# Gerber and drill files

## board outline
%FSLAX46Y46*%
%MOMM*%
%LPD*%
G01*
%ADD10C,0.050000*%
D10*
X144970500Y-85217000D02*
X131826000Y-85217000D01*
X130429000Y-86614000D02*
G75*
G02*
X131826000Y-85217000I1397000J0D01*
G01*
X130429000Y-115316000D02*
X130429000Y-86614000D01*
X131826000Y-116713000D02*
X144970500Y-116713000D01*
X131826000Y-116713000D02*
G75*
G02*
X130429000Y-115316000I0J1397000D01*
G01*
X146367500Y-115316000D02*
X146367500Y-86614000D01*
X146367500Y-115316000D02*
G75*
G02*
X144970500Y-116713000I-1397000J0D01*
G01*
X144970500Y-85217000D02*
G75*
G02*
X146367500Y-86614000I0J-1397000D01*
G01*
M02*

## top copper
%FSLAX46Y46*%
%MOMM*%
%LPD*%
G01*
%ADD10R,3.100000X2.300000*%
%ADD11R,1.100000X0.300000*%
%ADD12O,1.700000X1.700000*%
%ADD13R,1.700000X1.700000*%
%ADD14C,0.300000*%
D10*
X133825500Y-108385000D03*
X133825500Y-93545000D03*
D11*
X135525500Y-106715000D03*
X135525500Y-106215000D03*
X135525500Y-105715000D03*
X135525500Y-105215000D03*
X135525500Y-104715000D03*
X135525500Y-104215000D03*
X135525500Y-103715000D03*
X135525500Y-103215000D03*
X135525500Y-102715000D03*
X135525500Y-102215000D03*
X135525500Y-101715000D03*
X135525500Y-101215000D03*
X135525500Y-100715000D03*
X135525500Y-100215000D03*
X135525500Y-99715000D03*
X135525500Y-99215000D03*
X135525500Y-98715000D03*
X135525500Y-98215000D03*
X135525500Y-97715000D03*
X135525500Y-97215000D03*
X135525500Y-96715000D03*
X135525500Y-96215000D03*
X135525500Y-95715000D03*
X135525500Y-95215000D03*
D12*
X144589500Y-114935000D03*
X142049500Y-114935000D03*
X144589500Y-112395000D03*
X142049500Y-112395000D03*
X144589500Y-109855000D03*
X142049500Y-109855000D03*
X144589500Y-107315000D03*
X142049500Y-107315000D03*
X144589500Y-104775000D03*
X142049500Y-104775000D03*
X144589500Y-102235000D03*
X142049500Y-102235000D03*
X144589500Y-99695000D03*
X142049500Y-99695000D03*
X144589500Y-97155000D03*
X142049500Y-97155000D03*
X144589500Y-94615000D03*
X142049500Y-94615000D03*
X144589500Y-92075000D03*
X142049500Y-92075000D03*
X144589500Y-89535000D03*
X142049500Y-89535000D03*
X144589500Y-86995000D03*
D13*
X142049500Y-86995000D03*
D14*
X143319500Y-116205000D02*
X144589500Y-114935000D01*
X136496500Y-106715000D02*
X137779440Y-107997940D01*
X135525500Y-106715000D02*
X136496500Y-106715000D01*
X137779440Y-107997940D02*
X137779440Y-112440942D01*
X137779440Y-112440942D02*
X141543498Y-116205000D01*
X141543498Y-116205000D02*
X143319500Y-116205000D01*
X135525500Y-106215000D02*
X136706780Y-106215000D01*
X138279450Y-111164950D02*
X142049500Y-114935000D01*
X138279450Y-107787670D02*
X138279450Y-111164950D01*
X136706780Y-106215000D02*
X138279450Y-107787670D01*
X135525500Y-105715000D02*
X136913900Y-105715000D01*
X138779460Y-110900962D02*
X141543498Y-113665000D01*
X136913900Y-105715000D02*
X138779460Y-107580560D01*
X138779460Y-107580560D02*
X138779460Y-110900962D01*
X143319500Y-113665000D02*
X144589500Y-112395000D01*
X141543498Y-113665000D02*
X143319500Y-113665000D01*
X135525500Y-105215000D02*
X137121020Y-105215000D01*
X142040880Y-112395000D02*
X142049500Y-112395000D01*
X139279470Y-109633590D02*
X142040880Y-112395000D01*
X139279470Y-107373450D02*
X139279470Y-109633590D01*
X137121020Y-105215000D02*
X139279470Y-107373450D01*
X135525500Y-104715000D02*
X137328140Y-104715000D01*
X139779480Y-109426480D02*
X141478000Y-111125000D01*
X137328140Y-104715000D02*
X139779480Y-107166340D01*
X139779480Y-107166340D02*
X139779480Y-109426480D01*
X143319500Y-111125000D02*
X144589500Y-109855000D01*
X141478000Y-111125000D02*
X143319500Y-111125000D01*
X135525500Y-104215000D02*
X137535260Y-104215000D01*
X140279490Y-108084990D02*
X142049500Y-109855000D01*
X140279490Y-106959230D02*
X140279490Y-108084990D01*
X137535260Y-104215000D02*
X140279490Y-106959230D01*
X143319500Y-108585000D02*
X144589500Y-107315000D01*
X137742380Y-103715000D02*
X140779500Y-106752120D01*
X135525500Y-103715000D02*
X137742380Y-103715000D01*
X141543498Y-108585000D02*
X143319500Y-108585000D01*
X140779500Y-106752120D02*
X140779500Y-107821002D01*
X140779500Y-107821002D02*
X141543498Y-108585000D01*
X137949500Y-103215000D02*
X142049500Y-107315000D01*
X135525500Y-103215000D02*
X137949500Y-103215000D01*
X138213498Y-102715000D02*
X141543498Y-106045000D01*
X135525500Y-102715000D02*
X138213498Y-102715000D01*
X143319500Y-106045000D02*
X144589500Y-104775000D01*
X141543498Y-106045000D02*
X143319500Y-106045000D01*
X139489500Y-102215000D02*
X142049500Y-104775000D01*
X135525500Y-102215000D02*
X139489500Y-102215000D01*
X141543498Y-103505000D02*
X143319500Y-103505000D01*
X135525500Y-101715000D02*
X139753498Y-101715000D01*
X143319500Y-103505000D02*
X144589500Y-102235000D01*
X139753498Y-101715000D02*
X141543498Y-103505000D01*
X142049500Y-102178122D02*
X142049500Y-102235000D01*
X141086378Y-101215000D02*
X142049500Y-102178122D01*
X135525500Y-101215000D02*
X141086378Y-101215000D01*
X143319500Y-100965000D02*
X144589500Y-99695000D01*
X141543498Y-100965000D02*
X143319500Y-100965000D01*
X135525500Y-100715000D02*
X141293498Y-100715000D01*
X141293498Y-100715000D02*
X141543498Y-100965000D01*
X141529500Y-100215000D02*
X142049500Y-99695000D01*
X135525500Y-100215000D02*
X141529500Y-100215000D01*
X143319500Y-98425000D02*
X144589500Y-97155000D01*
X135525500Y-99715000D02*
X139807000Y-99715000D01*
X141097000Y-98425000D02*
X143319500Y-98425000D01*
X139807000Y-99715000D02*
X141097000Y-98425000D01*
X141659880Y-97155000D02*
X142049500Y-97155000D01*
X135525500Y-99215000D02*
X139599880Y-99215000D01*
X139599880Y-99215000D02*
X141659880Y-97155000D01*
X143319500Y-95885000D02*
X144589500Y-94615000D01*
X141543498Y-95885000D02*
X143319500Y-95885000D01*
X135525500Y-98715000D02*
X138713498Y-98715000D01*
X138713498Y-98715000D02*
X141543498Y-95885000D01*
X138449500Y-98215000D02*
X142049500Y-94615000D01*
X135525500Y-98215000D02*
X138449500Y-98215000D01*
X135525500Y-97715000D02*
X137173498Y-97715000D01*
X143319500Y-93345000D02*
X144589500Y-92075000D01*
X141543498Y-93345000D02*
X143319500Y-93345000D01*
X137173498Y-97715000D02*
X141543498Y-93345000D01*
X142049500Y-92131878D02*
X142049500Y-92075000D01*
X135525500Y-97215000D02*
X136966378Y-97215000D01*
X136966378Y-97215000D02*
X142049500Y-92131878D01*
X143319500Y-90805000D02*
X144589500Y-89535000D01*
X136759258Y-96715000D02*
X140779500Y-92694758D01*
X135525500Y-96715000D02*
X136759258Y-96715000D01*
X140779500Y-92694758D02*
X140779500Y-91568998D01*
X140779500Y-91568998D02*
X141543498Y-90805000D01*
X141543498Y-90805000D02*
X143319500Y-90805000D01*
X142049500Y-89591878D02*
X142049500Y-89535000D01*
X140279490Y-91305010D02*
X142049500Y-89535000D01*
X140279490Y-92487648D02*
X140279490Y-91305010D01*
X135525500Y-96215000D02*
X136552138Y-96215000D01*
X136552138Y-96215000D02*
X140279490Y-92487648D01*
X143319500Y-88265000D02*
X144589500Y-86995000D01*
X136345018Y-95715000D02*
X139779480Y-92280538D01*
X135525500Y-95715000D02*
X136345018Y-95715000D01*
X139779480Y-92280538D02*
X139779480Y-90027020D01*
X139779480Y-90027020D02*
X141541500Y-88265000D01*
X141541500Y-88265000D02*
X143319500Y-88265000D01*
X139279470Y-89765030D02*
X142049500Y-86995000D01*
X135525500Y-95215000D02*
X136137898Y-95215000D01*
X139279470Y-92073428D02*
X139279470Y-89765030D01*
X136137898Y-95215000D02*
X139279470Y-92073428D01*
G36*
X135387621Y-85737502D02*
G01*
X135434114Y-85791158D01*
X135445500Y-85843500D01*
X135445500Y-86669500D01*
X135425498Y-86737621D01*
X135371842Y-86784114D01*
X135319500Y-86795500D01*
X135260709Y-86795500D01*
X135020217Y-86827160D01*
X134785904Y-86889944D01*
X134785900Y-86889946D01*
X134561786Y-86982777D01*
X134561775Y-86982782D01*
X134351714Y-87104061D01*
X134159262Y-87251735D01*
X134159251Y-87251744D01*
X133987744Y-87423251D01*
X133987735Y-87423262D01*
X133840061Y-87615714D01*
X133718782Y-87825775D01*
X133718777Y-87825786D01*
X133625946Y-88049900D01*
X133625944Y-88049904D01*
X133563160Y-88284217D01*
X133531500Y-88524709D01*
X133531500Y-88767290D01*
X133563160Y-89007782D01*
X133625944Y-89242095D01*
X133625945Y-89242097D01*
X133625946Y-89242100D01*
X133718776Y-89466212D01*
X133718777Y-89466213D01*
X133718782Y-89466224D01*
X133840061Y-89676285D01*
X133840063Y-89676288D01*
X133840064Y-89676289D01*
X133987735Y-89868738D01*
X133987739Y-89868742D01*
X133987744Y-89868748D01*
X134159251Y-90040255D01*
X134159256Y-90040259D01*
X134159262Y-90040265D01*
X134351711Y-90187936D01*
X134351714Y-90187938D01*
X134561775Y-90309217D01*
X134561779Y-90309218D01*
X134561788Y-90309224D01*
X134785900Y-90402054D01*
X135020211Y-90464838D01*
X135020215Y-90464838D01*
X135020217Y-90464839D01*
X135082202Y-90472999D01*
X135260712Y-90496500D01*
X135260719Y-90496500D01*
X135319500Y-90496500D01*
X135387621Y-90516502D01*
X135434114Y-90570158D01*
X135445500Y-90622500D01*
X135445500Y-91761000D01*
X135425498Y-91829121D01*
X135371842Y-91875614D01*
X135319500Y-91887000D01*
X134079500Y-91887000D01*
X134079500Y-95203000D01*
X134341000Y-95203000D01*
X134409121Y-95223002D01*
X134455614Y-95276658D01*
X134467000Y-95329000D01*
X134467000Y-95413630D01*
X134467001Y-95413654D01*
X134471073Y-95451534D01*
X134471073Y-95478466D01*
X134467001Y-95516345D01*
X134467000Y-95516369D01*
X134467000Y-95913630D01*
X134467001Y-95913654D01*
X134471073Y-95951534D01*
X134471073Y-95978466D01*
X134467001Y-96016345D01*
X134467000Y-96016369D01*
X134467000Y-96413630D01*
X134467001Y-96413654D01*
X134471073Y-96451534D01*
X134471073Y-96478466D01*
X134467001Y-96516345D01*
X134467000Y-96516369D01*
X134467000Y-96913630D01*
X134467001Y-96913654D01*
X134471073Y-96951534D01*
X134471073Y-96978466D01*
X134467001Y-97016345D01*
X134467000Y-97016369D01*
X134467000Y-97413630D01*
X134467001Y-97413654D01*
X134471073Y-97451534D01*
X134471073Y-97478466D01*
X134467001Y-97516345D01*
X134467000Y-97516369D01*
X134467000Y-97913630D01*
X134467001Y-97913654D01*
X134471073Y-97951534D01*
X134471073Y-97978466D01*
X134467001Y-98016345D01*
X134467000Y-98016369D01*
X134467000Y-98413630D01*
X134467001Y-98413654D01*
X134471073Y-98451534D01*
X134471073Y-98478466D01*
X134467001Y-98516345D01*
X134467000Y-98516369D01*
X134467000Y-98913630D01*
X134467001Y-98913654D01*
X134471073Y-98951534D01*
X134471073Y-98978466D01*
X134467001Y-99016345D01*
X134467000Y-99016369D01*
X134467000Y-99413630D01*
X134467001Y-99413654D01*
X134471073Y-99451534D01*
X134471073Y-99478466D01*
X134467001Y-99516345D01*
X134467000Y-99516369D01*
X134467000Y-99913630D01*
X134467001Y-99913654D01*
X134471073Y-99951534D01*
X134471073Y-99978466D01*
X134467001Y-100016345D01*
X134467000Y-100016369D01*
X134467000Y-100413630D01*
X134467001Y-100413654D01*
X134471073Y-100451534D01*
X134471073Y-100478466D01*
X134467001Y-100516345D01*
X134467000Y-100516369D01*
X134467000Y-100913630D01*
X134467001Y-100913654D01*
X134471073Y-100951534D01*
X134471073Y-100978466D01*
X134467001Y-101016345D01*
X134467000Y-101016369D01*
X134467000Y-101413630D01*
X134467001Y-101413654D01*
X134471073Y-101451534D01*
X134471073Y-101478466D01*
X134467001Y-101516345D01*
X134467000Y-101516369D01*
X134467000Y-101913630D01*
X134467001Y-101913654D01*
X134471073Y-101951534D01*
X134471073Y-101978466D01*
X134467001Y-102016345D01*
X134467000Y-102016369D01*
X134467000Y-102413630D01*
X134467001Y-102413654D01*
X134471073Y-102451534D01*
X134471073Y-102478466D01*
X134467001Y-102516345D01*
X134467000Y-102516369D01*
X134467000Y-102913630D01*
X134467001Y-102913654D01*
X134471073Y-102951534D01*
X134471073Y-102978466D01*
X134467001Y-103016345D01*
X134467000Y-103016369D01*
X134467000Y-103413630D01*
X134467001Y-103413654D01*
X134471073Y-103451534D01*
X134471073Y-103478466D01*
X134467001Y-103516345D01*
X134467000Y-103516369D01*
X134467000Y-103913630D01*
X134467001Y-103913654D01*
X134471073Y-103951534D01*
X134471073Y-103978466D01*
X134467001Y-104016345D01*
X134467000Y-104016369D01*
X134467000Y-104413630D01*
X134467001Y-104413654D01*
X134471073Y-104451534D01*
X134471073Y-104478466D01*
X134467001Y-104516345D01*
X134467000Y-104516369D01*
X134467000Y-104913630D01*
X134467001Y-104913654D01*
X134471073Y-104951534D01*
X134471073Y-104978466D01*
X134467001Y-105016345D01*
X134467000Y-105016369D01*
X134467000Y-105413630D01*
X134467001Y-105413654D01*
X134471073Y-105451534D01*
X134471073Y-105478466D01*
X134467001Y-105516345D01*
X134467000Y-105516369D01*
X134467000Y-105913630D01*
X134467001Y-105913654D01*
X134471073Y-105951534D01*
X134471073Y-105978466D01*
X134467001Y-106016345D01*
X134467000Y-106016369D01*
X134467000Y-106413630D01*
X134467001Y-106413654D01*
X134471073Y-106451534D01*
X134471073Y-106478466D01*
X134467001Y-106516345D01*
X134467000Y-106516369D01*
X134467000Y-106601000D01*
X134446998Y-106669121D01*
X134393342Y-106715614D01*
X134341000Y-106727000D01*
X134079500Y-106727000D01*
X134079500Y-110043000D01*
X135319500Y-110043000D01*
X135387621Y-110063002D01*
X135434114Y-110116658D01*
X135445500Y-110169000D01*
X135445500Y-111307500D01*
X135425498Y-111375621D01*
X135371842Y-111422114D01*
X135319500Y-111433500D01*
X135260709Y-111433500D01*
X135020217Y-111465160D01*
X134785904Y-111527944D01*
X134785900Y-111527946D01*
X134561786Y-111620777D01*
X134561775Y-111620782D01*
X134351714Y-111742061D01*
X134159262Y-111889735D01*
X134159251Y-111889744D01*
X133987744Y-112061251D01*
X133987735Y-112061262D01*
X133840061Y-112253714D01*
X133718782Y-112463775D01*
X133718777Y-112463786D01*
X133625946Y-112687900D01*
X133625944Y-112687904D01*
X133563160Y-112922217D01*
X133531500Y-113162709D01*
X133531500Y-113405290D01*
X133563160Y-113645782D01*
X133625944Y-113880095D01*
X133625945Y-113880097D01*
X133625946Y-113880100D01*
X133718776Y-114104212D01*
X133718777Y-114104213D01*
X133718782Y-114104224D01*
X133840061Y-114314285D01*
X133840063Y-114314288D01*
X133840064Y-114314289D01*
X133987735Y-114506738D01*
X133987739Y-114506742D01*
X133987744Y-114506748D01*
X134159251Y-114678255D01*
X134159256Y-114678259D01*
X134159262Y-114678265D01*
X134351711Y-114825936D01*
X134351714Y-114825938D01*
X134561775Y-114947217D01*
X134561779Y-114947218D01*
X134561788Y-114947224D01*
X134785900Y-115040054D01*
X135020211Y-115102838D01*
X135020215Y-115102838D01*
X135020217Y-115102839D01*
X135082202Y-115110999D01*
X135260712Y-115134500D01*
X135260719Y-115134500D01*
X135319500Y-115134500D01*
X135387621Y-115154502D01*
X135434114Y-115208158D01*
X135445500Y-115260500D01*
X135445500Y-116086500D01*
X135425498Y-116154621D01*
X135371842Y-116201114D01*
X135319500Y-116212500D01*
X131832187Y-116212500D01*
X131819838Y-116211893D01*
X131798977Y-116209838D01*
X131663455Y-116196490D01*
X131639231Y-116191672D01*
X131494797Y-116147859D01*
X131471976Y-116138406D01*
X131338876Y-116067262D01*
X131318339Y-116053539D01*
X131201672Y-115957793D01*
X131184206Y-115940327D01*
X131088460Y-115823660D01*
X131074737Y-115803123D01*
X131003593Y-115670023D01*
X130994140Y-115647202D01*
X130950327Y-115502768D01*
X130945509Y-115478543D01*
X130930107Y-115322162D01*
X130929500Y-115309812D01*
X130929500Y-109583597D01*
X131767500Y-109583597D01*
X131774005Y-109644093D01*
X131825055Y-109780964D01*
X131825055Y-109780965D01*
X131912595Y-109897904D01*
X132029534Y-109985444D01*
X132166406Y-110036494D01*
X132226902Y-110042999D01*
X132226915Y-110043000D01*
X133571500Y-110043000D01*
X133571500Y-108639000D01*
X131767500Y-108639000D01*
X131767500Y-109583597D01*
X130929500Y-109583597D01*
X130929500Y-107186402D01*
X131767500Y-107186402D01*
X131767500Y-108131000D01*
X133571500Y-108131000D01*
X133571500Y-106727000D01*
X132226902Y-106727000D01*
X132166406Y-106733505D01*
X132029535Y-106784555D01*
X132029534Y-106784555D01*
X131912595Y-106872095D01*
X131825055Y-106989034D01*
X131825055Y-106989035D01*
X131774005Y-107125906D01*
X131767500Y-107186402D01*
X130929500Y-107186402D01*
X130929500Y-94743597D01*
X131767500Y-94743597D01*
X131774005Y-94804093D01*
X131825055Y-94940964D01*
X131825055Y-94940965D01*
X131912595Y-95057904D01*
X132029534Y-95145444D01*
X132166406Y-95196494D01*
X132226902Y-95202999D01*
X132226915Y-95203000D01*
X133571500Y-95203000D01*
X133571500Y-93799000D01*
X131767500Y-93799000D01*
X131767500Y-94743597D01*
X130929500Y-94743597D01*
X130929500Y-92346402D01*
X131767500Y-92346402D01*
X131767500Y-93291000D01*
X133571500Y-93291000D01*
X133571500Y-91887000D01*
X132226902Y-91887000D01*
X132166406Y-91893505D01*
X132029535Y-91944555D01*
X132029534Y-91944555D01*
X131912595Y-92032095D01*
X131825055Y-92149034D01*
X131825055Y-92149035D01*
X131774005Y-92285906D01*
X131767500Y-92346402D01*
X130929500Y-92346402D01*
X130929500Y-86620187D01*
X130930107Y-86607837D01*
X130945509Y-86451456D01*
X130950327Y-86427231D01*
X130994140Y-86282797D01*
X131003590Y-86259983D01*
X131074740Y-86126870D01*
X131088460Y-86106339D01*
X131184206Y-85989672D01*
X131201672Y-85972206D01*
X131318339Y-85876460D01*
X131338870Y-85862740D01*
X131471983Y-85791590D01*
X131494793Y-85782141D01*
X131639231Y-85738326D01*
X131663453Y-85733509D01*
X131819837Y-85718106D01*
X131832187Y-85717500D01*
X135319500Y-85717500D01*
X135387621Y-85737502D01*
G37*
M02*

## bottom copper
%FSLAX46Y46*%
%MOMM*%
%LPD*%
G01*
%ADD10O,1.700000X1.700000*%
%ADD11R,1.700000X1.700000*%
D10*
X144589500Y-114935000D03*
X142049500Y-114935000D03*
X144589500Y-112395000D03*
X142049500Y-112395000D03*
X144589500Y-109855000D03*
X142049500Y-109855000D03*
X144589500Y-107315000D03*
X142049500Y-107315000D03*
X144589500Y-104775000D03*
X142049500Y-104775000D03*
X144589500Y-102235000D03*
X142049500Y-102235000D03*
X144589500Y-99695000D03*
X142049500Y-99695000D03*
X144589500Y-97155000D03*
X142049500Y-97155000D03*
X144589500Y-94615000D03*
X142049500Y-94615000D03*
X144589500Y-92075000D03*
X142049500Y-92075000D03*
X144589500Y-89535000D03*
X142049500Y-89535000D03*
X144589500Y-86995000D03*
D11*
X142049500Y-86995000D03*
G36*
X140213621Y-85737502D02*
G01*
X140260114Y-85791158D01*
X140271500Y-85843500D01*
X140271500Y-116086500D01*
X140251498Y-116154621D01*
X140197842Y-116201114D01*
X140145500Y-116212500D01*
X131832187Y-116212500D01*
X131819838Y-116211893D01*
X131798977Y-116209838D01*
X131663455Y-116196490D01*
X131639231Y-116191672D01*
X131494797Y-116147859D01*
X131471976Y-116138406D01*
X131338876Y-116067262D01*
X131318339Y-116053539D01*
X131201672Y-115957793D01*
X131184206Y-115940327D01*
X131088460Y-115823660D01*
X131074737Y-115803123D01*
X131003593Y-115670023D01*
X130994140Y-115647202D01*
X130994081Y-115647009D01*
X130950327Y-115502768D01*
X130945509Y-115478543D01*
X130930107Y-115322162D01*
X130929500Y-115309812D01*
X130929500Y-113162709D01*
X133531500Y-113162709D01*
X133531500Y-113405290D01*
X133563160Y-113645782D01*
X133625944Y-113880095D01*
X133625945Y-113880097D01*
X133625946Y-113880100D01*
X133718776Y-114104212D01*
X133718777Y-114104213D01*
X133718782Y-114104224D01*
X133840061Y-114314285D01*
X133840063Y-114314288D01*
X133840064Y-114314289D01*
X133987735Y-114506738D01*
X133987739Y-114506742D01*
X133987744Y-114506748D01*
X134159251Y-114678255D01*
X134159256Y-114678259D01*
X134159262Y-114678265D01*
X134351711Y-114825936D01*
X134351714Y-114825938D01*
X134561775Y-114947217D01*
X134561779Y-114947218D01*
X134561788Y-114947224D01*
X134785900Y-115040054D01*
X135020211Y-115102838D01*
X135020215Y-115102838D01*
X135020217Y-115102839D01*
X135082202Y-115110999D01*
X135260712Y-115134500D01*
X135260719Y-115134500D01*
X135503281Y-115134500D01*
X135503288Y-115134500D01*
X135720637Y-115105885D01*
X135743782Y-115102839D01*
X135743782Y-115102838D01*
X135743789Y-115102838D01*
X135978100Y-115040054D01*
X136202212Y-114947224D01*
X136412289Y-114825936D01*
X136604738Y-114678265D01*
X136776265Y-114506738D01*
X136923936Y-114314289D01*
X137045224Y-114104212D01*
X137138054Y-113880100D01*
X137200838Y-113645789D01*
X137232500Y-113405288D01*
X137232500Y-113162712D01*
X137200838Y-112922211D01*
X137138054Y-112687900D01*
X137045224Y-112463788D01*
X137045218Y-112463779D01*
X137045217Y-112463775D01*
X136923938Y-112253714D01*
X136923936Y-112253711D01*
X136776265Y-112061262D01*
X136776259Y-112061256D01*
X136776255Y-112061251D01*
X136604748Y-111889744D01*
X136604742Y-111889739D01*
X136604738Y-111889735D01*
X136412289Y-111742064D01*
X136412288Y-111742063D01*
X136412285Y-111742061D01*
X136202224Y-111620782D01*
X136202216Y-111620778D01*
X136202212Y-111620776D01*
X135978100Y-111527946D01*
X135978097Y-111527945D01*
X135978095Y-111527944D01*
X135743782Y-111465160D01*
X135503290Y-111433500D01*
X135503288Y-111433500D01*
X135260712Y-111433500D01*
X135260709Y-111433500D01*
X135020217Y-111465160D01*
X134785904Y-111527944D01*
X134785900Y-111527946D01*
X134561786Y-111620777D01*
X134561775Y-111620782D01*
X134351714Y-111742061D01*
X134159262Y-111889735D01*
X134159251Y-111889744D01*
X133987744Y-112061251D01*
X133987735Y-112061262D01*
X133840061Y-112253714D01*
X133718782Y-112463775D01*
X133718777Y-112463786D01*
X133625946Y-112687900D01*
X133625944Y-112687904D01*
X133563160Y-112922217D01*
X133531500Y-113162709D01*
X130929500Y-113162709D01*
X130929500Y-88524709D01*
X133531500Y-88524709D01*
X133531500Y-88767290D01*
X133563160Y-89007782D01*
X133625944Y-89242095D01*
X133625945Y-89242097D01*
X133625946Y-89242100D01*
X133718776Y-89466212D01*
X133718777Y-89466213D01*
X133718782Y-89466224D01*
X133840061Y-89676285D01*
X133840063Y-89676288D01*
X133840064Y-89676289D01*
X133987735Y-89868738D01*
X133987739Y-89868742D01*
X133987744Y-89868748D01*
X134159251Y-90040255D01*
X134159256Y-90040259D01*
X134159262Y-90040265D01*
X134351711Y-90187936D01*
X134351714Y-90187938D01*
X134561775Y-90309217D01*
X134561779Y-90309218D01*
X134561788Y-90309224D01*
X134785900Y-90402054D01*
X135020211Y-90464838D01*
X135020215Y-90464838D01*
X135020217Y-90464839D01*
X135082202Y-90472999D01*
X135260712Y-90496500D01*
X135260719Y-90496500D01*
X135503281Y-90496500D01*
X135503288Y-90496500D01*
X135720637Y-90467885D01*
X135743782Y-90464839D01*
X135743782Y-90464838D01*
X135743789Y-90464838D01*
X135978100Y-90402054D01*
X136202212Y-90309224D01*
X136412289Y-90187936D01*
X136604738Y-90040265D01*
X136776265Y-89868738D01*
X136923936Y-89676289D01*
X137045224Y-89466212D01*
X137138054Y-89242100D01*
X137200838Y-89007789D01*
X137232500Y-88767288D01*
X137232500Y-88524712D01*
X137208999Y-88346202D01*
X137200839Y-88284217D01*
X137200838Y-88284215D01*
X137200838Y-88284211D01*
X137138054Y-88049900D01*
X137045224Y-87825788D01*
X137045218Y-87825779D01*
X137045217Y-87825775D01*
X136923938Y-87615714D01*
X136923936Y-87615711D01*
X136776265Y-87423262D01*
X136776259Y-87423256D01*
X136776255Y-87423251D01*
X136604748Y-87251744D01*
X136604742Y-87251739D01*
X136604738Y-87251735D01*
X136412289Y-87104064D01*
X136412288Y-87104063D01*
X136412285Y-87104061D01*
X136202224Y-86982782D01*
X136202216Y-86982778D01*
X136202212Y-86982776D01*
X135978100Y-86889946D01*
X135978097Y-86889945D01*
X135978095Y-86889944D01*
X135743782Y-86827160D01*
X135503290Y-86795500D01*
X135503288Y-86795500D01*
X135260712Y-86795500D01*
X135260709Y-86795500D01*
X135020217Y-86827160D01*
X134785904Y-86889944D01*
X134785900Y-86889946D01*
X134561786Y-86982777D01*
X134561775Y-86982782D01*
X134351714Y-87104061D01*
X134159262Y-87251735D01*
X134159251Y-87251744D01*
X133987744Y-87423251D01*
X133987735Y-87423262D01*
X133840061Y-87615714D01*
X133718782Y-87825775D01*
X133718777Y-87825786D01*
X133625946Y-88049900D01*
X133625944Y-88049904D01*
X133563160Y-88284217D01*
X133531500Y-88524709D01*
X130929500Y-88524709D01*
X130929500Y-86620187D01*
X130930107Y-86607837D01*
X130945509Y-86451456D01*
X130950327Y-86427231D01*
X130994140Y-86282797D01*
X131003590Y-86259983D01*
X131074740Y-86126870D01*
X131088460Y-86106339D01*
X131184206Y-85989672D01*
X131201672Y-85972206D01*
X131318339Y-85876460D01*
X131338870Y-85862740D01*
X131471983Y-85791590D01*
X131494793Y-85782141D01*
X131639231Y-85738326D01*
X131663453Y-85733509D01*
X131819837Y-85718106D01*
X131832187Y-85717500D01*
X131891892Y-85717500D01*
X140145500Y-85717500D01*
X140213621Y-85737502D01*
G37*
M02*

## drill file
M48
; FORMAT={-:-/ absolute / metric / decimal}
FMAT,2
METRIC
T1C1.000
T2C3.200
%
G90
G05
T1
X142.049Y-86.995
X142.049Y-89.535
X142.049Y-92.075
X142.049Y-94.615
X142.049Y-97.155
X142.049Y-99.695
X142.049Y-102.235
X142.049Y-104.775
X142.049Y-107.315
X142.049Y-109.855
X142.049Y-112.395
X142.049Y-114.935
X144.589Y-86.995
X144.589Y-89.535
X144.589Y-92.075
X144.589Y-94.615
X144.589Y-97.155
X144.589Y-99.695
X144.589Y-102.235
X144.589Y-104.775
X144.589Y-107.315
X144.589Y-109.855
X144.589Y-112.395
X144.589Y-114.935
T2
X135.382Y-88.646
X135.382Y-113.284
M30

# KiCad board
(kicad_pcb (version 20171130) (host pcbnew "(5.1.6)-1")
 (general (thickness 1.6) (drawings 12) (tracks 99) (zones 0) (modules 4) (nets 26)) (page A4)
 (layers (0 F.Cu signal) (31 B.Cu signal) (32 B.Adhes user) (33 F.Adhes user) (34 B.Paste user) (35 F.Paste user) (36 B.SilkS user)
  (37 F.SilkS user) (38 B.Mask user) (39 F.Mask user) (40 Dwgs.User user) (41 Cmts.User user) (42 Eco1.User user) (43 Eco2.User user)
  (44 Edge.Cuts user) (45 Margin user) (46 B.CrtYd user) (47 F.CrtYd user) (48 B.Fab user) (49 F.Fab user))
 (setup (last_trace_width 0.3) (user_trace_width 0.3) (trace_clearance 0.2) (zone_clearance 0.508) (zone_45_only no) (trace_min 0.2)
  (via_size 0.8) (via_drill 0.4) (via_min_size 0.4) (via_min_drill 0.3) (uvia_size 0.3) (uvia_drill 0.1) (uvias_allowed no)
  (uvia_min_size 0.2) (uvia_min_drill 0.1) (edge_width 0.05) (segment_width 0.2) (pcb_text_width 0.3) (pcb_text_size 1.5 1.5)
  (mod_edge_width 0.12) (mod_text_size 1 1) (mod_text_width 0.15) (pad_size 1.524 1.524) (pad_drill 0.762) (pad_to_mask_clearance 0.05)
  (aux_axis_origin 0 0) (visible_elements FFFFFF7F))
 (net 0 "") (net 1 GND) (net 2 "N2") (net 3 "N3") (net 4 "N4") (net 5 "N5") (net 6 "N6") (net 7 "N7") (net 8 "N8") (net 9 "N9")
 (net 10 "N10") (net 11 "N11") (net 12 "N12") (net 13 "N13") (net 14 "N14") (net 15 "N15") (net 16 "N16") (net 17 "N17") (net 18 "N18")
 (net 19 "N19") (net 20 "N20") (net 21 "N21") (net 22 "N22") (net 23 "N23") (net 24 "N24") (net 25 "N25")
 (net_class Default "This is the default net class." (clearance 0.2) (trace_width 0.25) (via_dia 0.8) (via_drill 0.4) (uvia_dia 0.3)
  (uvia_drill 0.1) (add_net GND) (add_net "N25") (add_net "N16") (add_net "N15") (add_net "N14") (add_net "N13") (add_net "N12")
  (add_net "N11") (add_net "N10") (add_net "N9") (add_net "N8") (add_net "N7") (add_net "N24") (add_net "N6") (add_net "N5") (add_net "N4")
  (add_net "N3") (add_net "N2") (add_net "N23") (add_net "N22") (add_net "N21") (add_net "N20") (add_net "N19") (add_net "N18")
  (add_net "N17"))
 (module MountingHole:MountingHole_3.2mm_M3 (layer F.Cu) (at 135.382 113.284)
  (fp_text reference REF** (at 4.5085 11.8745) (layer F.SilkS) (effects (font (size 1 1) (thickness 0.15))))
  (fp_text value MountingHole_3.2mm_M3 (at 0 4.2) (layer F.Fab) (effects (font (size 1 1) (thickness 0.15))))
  (pad 1 np_thru_hole circle (at 0 0) (size 3.2 3.2) (drill 3.2) (layers *.Cu *.Mask)))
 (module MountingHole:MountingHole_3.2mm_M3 (layer F.Cu) (at 135.382 88.646)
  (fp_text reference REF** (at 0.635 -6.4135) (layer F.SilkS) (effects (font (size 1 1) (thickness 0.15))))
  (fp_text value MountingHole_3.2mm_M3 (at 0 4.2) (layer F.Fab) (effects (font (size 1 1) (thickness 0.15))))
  (pad 1 np_thru_hole circle (at 0 0) (size 3.2 3.2) (drill 3.2) (layers *.Cu *.Mask)))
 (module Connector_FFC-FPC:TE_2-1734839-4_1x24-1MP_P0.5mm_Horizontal (layer F.Cu) (at 134.1755 100.965 270)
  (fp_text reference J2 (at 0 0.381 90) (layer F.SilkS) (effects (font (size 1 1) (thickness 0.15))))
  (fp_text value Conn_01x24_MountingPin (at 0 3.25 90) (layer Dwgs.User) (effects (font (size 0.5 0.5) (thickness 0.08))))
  (pad MP smd rect (at 7.42 0.35 270) (size 2.3 3.1) (layers F.Cu F.Paste F.Mask) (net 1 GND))
  (pad MP smd rect (at -7.42 0.35 270) (size 2.3 3.1) (layers F.Cu F.Paste F.Mask) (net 1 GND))
  (pad 24 smd rect (at 5.75 -1.35 270) (size 0.3 1.1) (layers F.Cu F.Paste F.Mask) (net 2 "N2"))
  (pad 23 smd rect (at 5.25 -1.35 270) (size 0.3 1.1) (layers F.Cu F.Paste F.Mask) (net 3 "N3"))
  (pad 22 smd rect (at 4.75 -1.35 270) (size 0.3 1.1) (layers F.Cu F.Paste F.Mask) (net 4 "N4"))
  (pad 21 smd rect (at 4.25 -1.35 270) (size 0.3 1.1) (layers F.Cu F.Paste F.Mask) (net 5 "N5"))
  (pad 20 smd rect (at 3.75 -1.35 270) (size 0.3 1.1) (layers F.Cu F.Paste F.Mask) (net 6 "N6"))
  (pad 19 smd rect (at 3.25 -1.35 270) (size 0.3 1.1) (layers F.Cu F.Paste F.Mask) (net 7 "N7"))
  (pad 18 smd rect (at 2.75 -1.35 270) (size 0.3 1.1) (layers F.Cu F.Paste F.Mask) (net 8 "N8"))
  (pad 17 smd rect (at 2.25 -1.35 270) (size 0.3 1.1) (layers F.Cu F.Paste F.Mask) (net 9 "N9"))
  (pad 16 smd rect (at 1.75 -1.35 270) (size 0.3 1.1) (layers F.Cu F.Paste F.Mask) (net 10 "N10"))
  (pad 15 smd rect (at 1.25 -1.35 270) (size 0.3 1.1) (layers F.Cu F.Paste F.Mask) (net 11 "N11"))
  (pad 14 smd rect (at 0.75 -1.35 270) (size 0.3 1.1) (layers F.Cu F.Paste F.Mask) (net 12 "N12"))
  (pad 13 smd rect (at 0.25 -1.35 270) (size 0.3 1.1) (layers F.Cu F.Paste F.Mask) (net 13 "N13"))
  (pad 12 smd rect (at -0.25 -1.35 270) (size 0.3 1.1) (layers F.Cu F.Paste F.Mask) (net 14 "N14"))
  (pad 11 smd rect (at -0.75 -1.35 270) (size 0.3 1.1) (layers F.Cu F.Paste F.Mask) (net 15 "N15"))
  (pad 10 smd rect (at -1.25 -1.35 270) (size 0.3 1.1) (layers F.Cu F.Paste F.Mask) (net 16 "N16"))
  (pad 9 smd rect (at -1.75 -1.35 270) (size 0.3 1.1) (layers F.Cu F.Paste F.Mask) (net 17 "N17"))
  (pad 8 smd rect (at -2.25 -1.35 270) (size 0.3 1.1) (layers F.Cu F.Paste F.Mask) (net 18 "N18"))
  (pad 7 smd rect (at -2.75 -1.35 270) (size 0.3 1.1) (layers F.Cu F.Paste F.Mask) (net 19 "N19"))
  (pad 6 smd rect (at -3.25 -1.35 270) (size 0.3 1.1) (layers F.Cu F.Paste F.Mask) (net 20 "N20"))
  (pad 5 smd rect (at -3.75 -1.35 270) (size 0.3 1.1) (layers F.Cu F.Paste F.Mask) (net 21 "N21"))
  (pad 4 smd rect (at -4.25 -1.35 270) (size 0.3 1.1) (layers F.Cu F.Paste F.Mask) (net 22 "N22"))
  (pad 3 smd rect (at -4.75 -1.35 270) (size 0.3 1.1) (layers F.Cu F.Paste F.Mask) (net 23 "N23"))
  (pad 2 smd rect (at -5.25 -1.35 270) (size 0.3 1.1) (layers F.Cu F.Paste F.Mask) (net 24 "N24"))
  (pad 1 smd rect (at -5.75 -1.35 270) (size 0.3 1.1) (layers F.Cu F.Paste F.Mask) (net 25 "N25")))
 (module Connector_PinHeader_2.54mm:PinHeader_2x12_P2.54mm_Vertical (layer F.Cu) (at 142.0495 86.995)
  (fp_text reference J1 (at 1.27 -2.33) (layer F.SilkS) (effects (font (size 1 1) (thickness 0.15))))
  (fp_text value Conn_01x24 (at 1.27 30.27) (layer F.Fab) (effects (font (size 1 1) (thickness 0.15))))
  (pad 24 thru_hole oval (at 2.54 27.94) (size 1.7 1.7) (drill 1) (layers *.Cu *.Mask) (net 2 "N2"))
  (pad 23 thru_hole oval (at 0 27.94) (size 1.7 1.7) (drill 1) (layers *.Cu *.Mask) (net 3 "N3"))
  (pad 22 thru_hole oval (at 2.54 25.4) (size 1.7 1.7) (drill 1) (layers *.Cu *.Mask) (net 4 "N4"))
  (pad 21 thru_hole oval (at 0 25.4) (size 1.7 1.7) (drill 1) (layers *.Cu *.Mask) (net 5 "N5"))
  (pad 20 thru_hole oval (at 2.54 22.86) (size 1.7 1.7) (drill 1) (layers *.Cu *.Mask) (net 6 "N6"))
  (pad 19 thru_hole oval (at 0 22.86) (size 1.7 1.7) (drill 1) (layers *.Cu *.Mask) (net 7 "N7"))
  (pad 18 thru_hole oval (at 2.54 20.32) (size 1.7 1.7) (drill 1) (layers *.Cu *.Mask) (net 8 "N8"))
  (pad 17 thru_hole oval (at 0 20.32) (size 1.7 1.7) (drill 1) (layers *.Cu *.Mask) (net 9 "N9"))
  (pad 16 thru_hole oval (at 2.54 17.78) (size 1.7 1.7) (drill 1) (layers *.Cu *.Mask) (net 10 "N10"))
  (pad 15 thru_hole oval (at 0 17.78) (size 1.7 1.7) (drill 1) (layers *.Cu *.Mask) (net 11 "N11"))
  (pad 14 thru_hole oval (at 2.54 15.24) (size 1.7 1.7) (drill 1) (layers *.Cu *.Mask) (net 12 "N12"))
  (pad 13 thru_hole oval (at 0 15.24) (size 1.7 1.7) (drill 1) (layers *.Cu *.Mask) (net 13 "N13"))
  (pad 12 thru_hole oval (at 2.54 12.7) (size 1.7 1.7) (drill 1) (layers *.Cu *.Mask) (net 14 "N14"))
  (pad 11 thru_hole oval (at 0 12.7) (size 1.7 1.7) (drill 1) (layers *.Cu *.Mask) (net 15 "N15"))
  (pad 10 thru_hole oval (at 2.54 10.16) (size 1.7 1.7) (drill 1) (layers *.Cu *.Mask) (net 16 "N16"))
  (pad 9 thru_hole oval (at 0 10.16) (size 1.7 1.7) (drill 1) (layers *.Cu *.Mask) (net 17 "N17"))
  (pad 8 thru_hole oval (at 2.54 7.62) (size 1.7 1.7) (drill 1) (layers *.Cu *.Mask) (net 18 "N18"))
  (pad 7 thru_hole oval (at 0 7.62) (size 1.7 1.7) (drill 1) (layers *.Cu *.Mask) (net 19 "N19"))
  (pad 6 thru_hole oval (at 2.54 5.08) (size 1.7 1.7) (drill 1) (layers *.Cu *.Mask) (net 20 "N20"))
  (pad 5 thru_hole oval (at 0 5.08) (size 1.7 1.7) (drill 1) (layers *.Cu *.Mask) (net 21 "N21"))
  (pad 4 thru_hole oval (at 2.54 2.54) (size 1.7 1.7) (drill 1) (layers *.Cu *.Mask) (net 22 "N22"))
  (pad 3 thru_hole oval (at 0 2.54) (size 1.7 1.7) (drill 1) (layers *.Cu *.Mask) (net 23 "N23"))
  (pad 2 thru_hole oval (at 2.54 0) (size 1.7 1.7) (drill 1) (layers *.Cu *.Mask) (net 24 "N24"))
  (pad 1 thru_hole rect (at 0 0) (size 1.7 1.7) (drill 1) (layers *.Cu *.Mask) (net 25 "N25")))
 (gr_line (start 144.9705 85.217) (end 131.826 85.217) (layer Edge.Cuts) (width 0.05))
 (gr_arc (start 131.826 86.614) (end 131.826 85.217) (angle -90) (layer Edge.Cuts) (width 0.05))
 (gr_line (start 130.429 115.316) (end 130.429 86.614) (layer Edge.Cuts) (width 0.05))
 (gr_line (start 131.826 116.713) (end 144.9705 116.713) (layer Edge.Cuts) (width 0.05))
 (gr_arc (start 131.826 115.316) (end 130.429 115.316) (angle -90) (layer Edge.Cuts) (width 0.05))
 (gr_line (start 146.3675 115.316) (end 146.3675 86.614) (layer Edge.Cuts) (width 0.05))
 (gr_arc (start 144.9705 115.316) (end 144.9705 116.713) (angle -90) (layer Edge.Cuts) (width 0.05))
 (gr_arc (start 144.9705 86.614) (end 146.3675 86.614) (angle -90) (layer Edge.Cuts) (width 0.05))
 (segment (start 143.3195 116.205) (end 144.5895 114.935) (width 0.3) (layer F.Cu) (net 2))
 (segment (start 136.4965 106.715) (end 137.77944 107.99794) (width 0.3) (layer F.Cu) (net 2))
 (segment (start 135.5255 106.715) (end 136.4965 106.715) (width 0.3) (layer F.Cu) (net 2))
 (segment (start 137.77944 107.99794) (end 137.77944 112.440942) (width 0.3) (layer F.Cu) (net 2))
 (segment (start 137.77944 112.440942) (end 141.543498 116.205) (width 0.3) (layer F.Cu) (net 2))
 (segment (start 141.543498 116.205) (end 143.3195 116.205) (width 0.3) (layer F.Cu) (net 2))
 (segment (start 135.5255 106.215) (end 136.70678 106.215) (width 0.3) (layer F.Cu) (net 3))
 (segment (start 138.27945 111.16495) (end 142.0495 114.935) (width 0.3) (layer F.Cu) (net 3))
 (segment (start 138.27945 107.78767) (end 138.27945 111.16495) (width 0.3) (layer F.Cu) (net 3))
 (segment (start 136.70678 106.215) (end 138.27945 107.78767) (width 0.3) (layer F.Cu) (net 3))
 (segment (start 135.5255 105.715) (end 136.9139 105.715) (width 0.3) (layer F.Cu) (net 4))
 (segment (start 138.77946 110.900962) (end 141.543498 113.665) (width 0.3) (layer F.Cu) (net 4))
 (segment (start 136.9139 105.715) (end 138.77946 107.58056) (width 0.3) (layer F.Cu) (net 4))
 (segment (start 138.77946 107.58056) (end 138.77946 110.900962) (width 0.3) (layer F.Cu) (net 4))
 (segment (start 143.3195 113.665) (end 144.5895 112.395) (width 0.3) (layer F.Cu) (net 4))
 (segment (start 141.543498 113.665) (end 143.3195 113.665) (width 0.3) (layer F.Cu) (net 4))
 (segment (start 135.5255 105.215) (end 137.12102 105.215) (width 0.3) (layer F.Cu) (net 5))
 (segment (start 142.04088 112.395) (end 142.0495 112.395) (width 0.3) (layer F.Cu) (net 5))
 (segment (start 139.27947 109.63359) (end 142.04088 112.395) (width 0.3) (layer F.Cu) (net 5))
 (segment (start 139.27947 107.37345) (end 139.27947 109.63359) (width 0.3) (layer F.Cu) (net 5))
 (segment (start 137.12102 105.215) (end 139.27947 107.37345) (width 0.3) (layer F.Cu) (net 5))
 (segment (start 135.5255 104.715) (end 137.32814 104.715) (width 0.3) (layer F.Cu) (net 6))
 (segment (start 139.77948 109.42648) (end 141.478 111.125) (width 0.3) (layer F.Cu) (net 6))
 (segment (start 137.32814 104.715) (end 139.77948 107.16634) (width 0.3) (layer F.Cu) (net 6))
 (segment (start 139.77948 107.16634) (end 139.77948 109.42648) (width 0.3) (layer F.Cu) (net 6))
 (segment (start 143.3195 111.125) (end 144.5895 109.855) (width 0.3) (layer F.Cu) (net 6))
 (segment (start 141.478 111.125) (end 143.3195 111.125) (width 0.3) (layer F.Cu) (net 6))
 (segment (start 135.5255 104.215) (end 137.53526 104.215) (width 0.3) (layer F.Cu) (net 7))
 (segment (start 140.27949 108.08499) (end 142.0495 109.855) (width 0.3) (layer F.Cu) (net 7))
 (segment (start 140.27949 106.95923) (end 140.27949 108.08499) (width 0.3) (layer F.Cu) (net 7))
 (segment (start 137.53526 104.215) (end 140.27949 106.95923) (width 0.3) (layer F.Cu) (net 7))
 (segment (start 143.3195 108.585) (end 144.5895 107.315) (width 0.3) (layer F.Cu) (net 8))
 (segment (start 137.74238 103.715) (end 140.7795 106.75212) (width 0.3) (layer F.Cu) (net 8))
 (segment (start 135.5255 103.715) (end 137.74238 103.715) (width 0.3) (layer F.Cu) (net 8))
 (segment (start 141.543498 108.585) (end 143.3195 108.585) (width 0.3) (layer F.Cu) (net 8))
 (segment (start 140.7795 106.75212) (end 140.7795 107.821002) (width 0.3) (layer F.Cu) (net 8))
 (segment (start 140.7795 107.821002) (end 141.543498 108.585) (width 0.3) (layer F.Cu) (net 8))
 (segment (start 137.9495 103.215) (end 142.0495 107.315) (width 0.3) (layer F.Cu) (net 9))
 (segment (start 135.5255 103.215) (end 137.9495 103.215) (width 0.3) (layer F.Cu) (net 9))
 (segment (start 138.213498 102.715) (end 141.543498 106.045) (width 0.3) (layer F.Cu) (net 10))
 (segment (start 135.5255 102.715) (end 138.213498 102.715) (width 0.3) (layer F.Cu) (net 10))
 (segment (start 143.3195 106.045) (end 144.5895 104.775) (width 0.3) (layer F.Cu) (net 10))
 (segment (start 141.543498 106.045) (end 143.3195 106.045) (width 0.3) (layer F.Cu) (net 10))
 (segment (start 139.4895 102.215) (end 142.0495 104.775) (width 0.3) (layer F.Cu) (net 11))
 (segment (start 135.5255 102.215) (end 139.4895 102.215) (width 0.3) (layer F.Cu) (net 11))
 (segment (start 141.543498 103.505) (end 143.3195 103.505) (width 0.3) (layer F.Cu) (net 12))
 (segment (start 135.5255 101.715) (end 139.753498 101.715) (width 0.3) (layer F.Cu) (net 12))
 (segment (start 143.3195 103.505) (end 144.5895 102.235) (width 0.3) (layer F.Cu) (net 12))
 (segment (start 139.753498 101.715) (end 141.543498 103.505) (width 0.3) (layer F.Cu) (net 12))
 (segment (start 142.0495 102.178122) (end 142.0495 102.235) (width 0.3) (layer F.Cu) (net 13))
 (segment (start 141.086378 101.215) (end 142.0495 102.178122) (width 0.3) (layer F.Cu) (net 13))
 (segment (start 135.5255 101.215) (end 141.086378 101.215) (width 0.3) (layer F.Cu) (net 13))
 (segment (start 143.3195 100.965) (end 144.5895 99.695) (width 0.3) (layer F.Cu) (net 14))
 (segment (start 141.543498 100.965) (end 143.3195 100.965) (width 0.3) (layer F.Cu) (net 14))
 (segment (start 135.5255 100.715) (end 141.293498 100.715) (width 0.3) (layer F.Cu) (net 14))
 (segment (start 141.293498 100.715) (end 141.543498 100.965) (width 0.3) (layer F.Cu) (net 14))
 (segment (start 141.5295 100.215) (end 142.0495 99.695) (width 0.3) (layer F.Cu) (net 15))
 (segment (start 135.5255 100.215) (end 141.5295 100.215) (width 0.3) (layer F.Cu) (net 15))
 (segment (start 143.3195 98.425) (end 144.5895 97.155) (width 0.3) (layer F.Cu) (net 16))
 (segment (start 135.5255 99.715) (end 139.807 99.715) (width 0.3) (layer F.Cu) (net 16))
 (segment (start 141.097 98.425) (end 143.3195 98.425) (width 0.3) (layer F.Cu) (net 16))
 (segment (start 139.807 99.715) (end 141.097 98.425) (width 0.3) (layer F.Cu) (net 16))
 (segment (start 141.65988 97.155) (end 142.0495 97.155) (width 0.3) (layer F.Cu) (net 17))
 (segment (start 135.5255 99.215) (end 139.59988 99.215) (width 0.3) (layer F.Cu) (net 17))
 (segment (start 139.59988 99.215) (end 141.65988 97.155) (width 0.3) (layer F.Cu) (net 17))
 (segment (start 143.3195 95.885) (end 144.5895 94.615) (width 0.3) (layer F.Cu) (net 18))
 (segment (start 141.543498 95.885) (end 143.3195 95.885) (width 0.3) (layer F.Cu) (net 18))
 (segment (start 135.5255 98.715) (end 138.713498 98.715) (width 0.3) (layer F.Cu) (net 18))
 (segment (start 138.713498 98.715) (end 141.543498 95.885) (width 0.3) (layer F.Cu) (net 18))
 (segment (start 138.4495 98.215) (end 142.0495 94.615) (width 0.3) (layer F.Cu) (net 19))
 (segment (start 135.5255 98.215) (end 138.4495 98.215) (width 0.3) (layer F.Cu) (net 19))
 (segment (start 135.5255 97.715) (end 137.173498 97.715) (width 0.3) (layer F.Cu) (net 20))
 (segment (start 143.3195 93.345) (end 144.5895 92.075) (width 0.3) (layer F.Cu) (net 20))
 (segment (start 141.543498 93.345) (end 143.3195 93.345) (width 0.3) (layer F.Cu) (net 20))
 (segment (start 137.173498 97.715) (end 141.543498 93.345) (width 0.3) (layer F.Cu) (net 20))
 (segment (start 142.0495 92.131878) (end 142.0495 92.075) (width 0.3) (layer F.Cu) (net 21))
 (segment (start 135.5255 97.215) (end 136.966378 97.215) (width 0.3) (layer F.Cu) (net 21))
 (segment (start 136.966378 97.215) (end 142.0495 92.131878) (width 0.3) (layer F.Cu) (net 21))
 (segment (start 143.3195 90.805) (end 144.5895 89.535) (width 0.3) (layer F.Cu) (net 22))
 (segment (start 136.759258 96.715) (end 140.7795 92.694758) (width 0.3) (layer F.Cu) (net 22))
 (segment (start 135.5255 96.715) (end 136.759258 96.715) (width 0.3) (layer F.Cu) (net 22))
 (segment (start 140.7795 92.694758) (end 140.7795 91.568998) (width 0.3) (layer F.Cu) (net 22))
 (segment (start 140.7795 91.568998) (end 141.543498 90.805) (width 0.3) (layer F.Cu) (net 22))
 (segment (start 141.543498 90.805) (end 143.3195 90.805) (width 0.3) (layer F.Cu) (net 22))
 (segment (start 142.0495 89.591878) (end 142.0495 89.535) (width 0.3) (layer F.Cu) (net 23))
 (segment (start 140.27949 91.30501) (end 142.0495 89.535) (width 0.3) (layer F.Cu) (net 23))
 (segment (start 140.27949 92.487648) (end 140.27949 91.30501) (width 0.3) (layer F.Cu) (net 23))
 (segment (start 135.5255 96.215) (end 136.552138 96.215) (width 0.3) (layer F.Cu) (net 23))
 (segment (start 136.552138 96.215) (end 140.27949 92.487648) (width 0.3) (layer F.Cu) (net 23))
 (segment (start 143.3195 88.265) (end 144.5895 86.995) (width 0.3) (layer F.Cu) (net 24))
 (segment (start 136.345018 95.715) (end 139.77948 92.280538) (width 0.3) (layer F.Cu) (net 24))
 (segment (start 135.5255 95.715) (end 136.345018 95.715) (width 0.3) (layer F.Cu) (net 24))
 (segment (start 139.77948 92.280538) (end 139.77948 90.02702) (width 0.3) (layer F.Cu) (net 24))
 (segment (start 139.77948 90.02702) (end 141.5415 88.265) (width 0.3) (layer F.Cu) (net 24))
 (segment (start 141.5415 88.265) (end 143.3195 88.265) (width 0.3) (layer F.Cu) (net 24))
 (segment (start 139.27947 89.76503) (end 142.0495 86.995) (width 0.3) (layer F.Cu) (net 25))
 (segment (start 135.5255 95.215) (end 136.137898 95.215) (width 0.3) (layer F.Cu) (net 25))
 (segment (start 139.27947 92.073428) (end 139.27947 89.76503) (width 0.3) (layer F.Cu) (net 25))
 (segment (start 136.137898 95.215) (end 139.27947 92.073428) (width 0.3) (layer F.Cu) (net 25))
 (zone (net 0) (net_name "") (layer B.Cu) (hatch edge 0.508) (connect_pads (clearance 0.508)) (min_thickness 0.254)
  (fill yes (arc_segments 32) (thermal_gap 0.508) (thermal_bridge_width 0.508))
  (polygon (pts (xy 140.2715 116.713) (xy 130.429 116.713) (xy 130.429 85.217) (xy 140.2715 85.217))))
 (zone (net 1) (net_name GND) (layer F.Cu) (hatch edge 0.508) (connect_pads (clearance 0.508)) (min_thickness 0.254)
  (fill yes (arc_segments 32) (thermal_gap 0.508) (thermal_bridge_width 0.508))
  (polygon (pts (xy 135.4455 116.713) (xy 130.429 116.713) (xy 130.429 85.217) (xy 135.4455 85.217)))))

